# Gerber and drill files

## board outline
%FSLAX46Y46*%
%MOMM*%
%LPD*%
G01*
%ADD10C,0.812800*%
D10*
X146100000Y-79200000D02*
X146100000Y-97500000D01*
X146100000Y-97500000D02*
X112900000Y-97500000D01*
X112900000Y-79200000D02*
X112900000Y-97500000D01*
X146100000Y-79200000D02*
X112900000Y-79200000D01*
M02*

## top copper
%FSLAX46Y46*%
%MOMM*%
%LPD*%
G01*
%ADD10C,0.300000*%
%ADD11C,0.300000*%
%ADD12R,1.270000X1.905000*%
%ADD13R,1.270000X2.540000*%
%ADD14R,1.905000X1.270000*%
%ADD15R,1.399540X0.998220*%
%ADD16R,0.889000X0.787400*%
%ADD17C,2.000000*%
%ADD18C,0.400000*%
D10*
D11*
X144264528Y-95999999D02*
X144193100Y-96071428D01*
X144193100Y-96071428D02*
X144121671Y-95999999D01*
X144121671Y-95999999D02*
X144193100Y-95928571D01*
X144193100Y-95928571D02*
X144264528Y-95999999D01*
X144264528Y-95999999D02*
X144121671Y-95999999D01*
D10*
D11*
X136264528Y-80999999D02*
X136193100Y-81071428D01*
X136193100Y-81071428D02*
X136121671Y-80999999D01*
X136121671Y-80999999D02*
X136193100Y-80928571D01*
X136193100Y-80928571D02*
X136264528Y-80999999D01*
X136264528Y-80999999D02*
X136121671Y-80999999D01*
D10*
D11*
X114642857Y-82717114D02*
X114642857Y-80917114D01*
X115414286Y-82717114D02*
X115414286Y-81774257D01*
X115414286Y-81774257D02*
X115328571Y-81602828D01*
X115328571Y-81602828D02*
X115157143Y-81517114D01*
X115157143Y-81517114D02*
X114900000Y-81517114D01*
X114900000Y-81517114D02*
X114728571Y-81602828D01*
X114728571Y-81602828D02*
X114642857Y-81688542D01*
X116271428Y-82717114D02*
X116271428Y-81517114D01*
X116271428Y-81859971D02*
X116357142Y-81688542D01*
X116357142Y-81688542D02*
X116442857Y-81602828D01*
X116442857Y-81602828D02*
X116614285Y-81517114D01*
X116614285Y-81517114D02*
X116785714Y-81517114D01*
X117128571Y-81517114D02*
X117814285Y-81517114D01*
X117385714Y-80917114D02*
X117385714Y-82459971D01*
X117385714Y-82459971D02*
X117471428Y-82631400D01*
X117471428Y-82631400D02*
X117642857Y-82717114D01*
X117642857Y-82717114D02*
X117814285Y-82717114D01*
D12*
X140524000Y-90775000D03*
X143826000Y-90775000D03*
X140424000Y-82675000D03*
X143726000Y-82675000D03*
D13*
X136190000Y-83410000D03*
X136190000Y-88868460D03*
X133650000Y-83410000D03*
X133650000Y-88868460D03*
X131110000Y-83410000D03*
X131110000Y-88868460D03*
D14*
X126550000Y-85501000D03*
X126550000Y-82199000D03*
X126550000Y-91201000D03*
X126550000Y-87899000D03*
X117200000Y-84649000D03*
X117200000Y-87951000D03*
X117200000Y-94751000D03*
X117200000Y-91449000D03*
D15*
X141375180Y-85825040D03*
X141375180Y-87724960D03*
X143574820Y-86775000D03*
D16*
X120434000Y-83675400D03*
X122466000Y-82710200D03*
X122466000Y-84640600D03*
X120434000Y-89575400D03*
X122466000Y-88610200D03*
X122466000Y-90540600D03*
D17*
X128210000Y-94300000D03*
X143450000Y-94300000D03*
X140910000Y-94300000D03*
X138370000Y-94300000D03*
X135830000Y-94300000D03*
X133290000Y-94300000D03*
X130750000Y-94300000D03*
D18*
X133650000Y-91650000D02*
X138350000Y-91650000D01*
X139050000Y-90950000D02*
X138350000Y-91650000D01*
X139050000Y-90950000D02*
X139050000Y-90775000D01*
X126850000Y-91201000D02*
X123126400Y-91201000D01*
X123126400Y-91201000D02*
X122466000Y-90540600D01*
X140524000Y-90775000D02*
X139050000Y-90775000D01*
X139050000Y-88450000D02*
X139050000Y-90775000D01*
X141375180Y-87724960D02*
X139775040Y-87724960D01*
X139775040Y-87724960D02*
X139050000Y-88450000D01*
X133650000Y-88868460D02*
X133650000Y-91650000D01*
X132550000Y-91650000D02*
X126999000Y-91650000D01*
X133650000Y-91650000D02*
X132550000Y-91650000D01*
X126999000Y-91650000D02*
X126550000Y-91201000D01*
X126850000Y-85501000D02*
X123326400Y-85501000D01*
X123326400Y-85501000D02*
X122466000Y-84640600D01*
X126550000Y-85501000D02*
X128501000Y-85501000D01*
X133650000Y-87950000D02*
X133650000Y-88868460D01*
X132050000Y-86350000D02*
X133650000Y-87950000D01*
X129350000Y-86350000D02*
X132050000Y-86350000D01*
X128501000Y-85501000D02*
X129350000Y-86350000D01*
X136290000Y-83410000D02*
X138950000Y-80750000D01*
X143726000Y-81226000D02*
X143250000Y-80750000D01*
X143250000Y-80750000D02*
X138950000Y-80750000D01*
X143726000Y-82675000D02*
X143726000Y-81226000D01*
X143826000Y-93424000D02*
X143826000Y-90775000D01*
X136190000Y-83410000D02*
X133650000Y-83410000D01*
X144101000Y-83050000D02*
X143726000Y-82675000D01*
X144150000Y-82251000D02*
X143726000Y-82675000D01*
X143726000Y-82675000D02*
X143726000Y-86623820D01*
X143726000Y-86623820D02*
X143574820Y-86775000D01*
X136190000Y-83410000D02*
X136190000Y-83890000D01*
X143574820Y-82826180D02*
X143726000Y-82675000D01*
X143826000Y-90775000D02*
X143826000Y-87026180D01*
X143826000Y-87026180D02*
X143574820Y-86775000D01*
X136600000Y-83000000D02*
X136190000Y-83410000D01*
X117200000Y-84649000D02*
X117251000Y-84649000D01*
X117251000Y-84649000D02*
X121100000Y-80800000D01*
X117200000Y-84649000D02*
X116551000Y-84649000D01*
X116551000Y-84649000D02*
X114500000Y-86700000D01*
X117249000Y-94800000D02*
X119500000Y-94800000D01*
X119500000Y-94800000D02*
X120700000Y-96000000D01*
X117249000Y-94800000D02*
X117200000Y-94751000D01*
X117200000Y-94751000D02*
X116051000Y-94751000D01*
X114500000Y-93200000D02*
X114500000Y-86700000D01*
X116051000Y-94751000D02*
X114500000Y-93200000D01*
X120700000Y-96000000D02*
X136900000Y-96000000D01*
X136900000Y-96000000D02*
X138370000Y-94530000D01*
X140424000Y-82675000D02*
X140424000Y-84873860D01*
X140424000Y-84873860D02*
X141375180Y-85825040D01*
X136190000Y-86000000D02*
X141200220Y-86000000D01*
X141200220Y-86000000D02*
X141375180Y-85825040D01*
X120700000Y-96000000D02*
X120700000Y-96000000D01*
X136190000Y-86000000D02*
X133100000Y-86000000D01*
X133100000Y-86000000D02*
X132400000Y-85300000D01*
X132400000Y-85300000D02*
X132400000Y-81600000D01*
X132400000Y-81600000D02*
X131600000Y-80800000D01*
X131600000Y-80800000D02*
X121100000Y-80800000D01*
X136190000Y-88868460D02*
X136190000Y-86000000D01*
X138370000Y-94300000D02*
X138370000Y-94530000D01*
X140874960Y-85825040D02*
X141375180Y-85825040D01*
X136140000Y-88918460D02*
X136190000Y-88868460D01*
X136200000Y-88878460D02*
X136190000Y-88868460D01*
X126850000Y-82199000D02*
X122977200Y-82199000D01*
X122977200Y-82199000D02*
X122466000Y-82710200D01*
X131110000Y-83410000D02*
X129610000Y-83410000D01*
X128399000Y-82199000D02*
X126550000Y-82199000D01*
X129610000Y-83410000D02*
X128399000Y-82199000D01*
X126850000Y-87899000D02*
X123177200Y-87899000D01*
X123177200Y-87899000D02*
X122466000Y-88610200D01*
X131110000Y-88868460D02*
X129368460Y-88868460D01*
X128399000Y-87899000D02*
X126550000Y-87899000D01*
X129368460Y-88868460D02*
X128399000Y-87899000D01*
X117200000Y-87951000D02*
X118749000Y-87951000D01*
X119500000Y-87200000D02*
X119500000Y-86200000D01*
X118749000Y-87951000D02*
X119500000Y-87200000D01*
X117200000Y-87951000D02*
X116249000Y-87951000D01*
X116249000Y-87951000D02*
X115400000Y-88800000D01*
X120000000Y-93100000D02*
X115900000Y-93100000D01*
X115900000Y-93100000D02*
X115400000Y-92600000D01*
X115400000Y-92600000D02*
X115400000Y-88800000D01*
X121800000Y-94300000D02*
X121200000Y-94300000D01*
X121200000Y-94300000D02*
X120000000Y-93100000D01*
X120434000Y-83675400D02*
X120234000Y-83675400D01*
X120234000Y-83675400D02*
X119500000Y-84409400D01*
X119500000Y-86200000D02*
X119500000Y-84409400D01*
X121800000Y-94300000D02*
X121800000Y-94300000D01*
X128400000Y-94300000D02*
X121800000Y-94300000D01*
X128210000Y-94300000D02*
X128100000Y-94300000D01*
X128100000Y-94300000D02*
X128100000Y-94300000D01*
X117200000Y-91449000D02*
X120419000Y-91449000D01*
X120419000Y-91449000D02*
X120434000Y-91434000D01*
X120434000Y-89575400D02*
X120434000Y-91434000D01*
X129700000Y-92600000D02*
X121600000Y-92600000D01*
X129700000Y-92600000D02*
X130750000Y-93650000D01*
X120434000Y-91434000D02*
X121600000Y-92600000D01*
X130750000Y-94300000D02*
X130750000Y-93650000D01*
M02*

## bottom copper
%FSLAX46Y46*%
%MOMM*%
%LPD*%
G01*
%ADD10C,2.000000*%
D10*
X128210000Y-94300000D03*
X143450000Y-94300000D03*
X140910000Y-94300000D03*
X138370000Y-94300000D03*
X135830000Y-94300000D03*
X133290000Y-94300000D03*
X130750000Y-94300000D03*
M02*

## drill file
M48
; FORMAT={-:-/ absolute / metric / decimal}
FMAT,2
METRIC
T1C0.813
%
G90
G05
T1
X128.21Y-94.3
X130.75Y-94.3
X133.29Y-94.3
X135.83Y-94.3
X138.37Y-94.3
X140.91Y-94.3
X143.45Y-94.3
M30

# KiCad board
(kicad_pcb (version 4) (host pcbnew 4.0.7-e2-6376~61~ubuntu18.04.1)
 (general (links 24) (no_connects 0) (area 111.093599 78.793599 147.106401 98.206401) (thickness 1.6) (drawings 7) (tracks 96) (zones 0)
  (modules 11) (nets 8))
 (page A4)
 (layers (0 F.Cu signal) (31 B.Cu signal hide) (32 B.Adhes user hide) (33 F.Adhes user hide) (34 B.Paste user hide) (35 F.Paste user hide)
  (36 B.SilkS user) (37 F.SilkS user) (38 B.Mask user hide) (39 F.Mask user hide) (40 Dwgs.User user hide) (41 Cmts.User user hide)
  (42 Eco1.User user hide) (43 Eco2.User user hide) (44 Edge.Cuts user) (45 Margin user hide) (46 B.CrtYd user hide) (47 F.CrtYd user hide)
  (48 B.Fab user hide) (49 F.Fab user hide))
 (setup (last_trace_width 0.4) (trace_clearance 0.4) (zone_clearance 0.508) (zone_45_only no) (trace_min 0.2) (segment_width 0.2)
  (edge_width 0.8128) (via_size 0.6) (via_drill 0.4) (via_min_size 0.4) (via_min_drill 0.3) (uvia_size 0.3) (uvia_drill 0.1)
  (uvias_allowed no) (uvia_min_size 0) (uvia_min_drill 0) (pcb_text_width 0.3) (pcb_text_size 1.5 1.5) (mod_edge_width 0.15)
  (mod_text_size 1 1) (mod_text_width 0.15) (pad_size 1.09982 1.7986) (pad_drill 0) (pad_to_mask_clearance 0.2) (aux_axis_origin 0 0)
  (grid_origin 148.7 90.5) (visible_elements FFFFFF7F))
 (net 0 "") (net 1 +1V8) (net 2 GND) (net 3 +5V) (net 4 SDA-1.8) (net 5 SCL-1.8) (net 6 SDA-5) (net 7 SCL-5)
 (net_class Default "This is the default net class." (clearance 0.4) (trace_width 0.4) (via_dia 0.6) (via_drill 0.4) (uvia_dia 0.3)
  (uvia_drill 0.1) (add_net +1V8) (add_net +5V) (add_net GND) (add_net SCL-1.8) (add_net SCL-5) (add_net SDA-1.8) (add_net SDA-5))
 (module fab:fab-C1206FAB (layer F.Cu) (at 142.175 90.775)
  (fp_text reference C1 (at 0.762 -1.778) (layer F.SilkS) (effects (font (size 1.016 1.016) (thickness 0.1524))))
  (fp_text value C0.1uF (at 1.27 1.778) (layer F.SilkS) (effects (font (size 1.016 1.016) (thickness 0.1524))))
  (pad 1 smd rect (at -1.651 0) (size 1.27 1.905) (layers F.Cu F.Paste F.Mask) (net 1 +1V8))
  (pad 2 smd rect (at 1.651 0) (size 1.27 1.905) (layers F.Cu F.Paste F.Mask) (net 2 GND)))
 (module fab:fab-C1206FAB (layer F.Cu) (at 142.075 82.675)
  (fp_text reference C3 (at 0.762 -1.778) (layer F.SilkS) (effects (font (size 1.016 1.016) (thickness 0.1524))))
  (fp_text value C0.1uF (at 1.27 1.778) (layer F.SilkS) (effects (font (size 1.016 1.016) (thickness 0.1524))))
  (pad 1 smd rect (at -1.651 0) (size 1.27 1.905) (layers F.Cu F.Paste F.Mask) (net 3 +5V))
  (pad 2 smd rect (at 1.651 0) (size 1.27 1.905) (layers F.Cu F.Paste F.Mask) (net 2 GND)))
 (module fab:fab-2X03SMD (layer F.Cu) (at 133.65 85.95 270)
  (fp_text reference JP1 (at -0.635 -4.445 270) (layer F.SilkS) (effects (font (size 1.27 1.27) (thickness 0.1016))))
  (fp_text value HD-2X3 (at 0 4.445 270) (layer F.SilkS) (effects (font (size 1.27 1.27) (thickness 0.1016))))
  (pad 1 smd rect (at -2.54 -2.54 270) (size 2.54 1.27) (layers F.Cu F.Paste F.Mask) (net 2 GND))
  (pad 2 smd rect (at 2.91846 -2.54 270) (size 2.54 1.27) (layers F.Cu F.Paste F.Mask) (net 3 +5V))
  (pad 3 smd rect (at -2.54 0 270) (size 2.54 1.27) (layers F.Cu F.Paste F.Mask) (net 2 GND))
  (pad 4 smd rect (at 2.91846 0 270) (size 2.54 1.27) (layers F.Cu F.Paste F.Mask) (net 1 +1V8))
  (pad 5 smd rect (at -2.54 2.54 270) (size 2.54 1.27) (layers F.Cu F.Paste F.Mask) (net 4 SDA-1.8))
  (pad 6 smd rect (at 2.91846 2.54 270) (size 2.54 1.27) (layers F.Cu F.Paste F.Mask) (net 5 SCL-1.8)))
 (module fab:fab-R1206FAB (layer F.Cu) (at 126.55 83.85 90)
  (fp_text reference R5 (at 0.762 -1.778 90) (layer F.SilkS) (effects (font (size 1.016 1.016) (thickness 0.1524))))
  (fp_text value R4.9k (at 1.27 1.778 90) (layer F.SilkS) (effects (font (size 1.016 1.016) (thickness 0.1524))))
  (pad 1 smd rect (at -1.651 0 90) (size 1.27 1.905) (layers F.Cu F.Paste F.Mask) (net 1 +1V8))
  (pad 2 smd rect (at 1.651 0 90) (size 1.27 1.905) (layers F.Cu F.Paste F.Mask) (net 4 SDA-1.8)))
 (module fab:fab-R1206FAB (layer F.Cu) (at 126.55 89.55 90)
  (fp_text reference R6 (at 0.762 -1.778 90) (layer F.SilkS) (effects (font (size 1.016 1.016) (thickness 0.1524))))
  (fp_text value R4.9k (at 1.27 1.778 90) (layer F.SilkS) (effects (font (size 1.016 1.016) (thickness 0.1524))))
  (pad 1 smd rect (at -1.651 0 90) (size 1.27 1.905) (layers F.Cu F.Paste F.Mask) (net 1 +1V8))
  (pad 2 smd rect (at 1.651 0 90) (size 1.27 1.905) (layers F.Cu F.Paste F.Mask) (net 5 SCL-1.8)))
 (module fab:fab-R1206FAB (layer F.Cu) (at 117.2 86.3 270)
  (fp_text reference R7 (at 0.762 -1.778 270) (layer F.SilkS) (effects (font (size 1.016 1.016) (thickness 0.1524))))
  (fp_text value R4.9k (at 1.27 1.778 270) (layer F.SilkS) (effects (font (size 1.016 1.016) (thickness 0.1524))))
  (pad 1 smd rect (at -1.651 0 270) (size 1.27 1.905) (layers F.Cu F.Paste F.Mask) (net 3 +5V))
  (pad 2 smd rect (at 1.651 0 270) (size 1.27 1.905) (layers F.Cu F.Paste F.Mask) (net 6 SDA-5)))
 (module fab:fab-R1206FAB (layer F.Cu) (at 117.2 93.1 90)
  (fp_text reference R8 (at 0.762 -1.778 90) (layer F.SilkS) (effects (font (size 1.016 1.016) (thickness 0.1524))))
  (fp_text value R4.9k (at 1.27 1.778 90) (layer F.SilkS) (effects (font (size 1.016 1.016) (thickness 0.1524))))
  (pad 1 smd rect (at -1.651 0 90) (size 1.27 1.905) (layers F.Cu F.Paste F.Mask) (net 3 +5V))
  (pad 2 smd rect (at 1.651 0 90) (size 1.27 1.905) (layers F.Cu F.Paste F.Mask) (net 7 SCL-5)))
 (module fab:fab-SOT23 (layer F.Cu) (at 142.475 86.775 270)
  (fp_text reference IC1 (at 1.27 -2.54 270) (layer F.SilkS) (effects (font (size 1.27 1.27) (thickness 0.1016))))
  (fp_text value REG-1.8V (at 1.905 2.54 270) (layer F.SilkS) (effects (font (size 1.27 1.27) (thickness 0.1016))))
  (pad 1 smd rect (at -0.94996 1.09982 270) (size 0.99822 1.39954) (layers F.Cu F.Paste F.Mask) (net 3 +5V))
  (pad 2 smd rect (at 0.94996 1.09982 270) (size 0.99822 1.39954) (layers F.Cu F.Paste F.Mask) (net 1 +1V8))
  (pad 3 smd rect (at 0 -1.09982 270) (size 0.99822 1.39954) (layers F.Cu F.Paste F.Mask) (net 2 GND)))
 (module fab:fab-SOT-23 (layer F.Cu) (at 121.45 83.65 270)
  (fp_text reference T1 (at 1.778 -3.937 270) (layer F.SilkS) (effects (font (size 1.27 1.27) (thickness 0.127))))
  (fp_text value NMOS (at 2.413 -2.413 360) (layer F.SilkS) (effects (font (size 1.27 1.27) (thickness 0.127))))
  (pad 1 smd rect (at 0.0254 1.016 270) (size 0.7874 0.889) (layers F.Cu F.Paste F.Mask) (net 6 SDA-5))
  (pad 2 smd rect (at -0.9398 -1.016 270) (size 0.7874 0.889) (layers F.Cu F.Paste F.Mask) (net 4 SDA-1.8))
  (pad 3 smd rect (at 0.9906 -1.016 270) (size 0.7874 0.889) (layers F.Cu F.Paste F.Mask) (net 1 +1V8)))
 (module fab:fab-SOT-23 (layer F.Cu) (at 121.45 89.55 270)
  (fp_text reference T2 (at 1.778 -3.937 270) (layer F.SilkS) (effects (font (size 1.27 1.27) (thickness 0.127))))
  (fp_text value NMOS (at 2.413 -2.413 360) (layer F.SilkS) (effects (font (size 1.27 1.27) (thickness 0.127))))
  (pad 1 smd rect (at 0.0254 1.016 270) (size 0.7874 0.889) (layers F.Cu F.Paste F.Mask) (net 7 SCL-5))
  (pad 2 smd rect (at -0.9398 -1.016 270) (size 0.7874 0.889) (layers F.Cu F.Paste F.Mask) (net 5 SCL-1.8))
  (pad 3 smd rect (at 0.9906 -1.016 270) (size 0.7874 0.889) (layers F.Cu F.Paste F.Mask) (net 1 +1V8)))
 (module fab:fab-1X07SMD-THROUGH (layer F.Cu) (at 137.1 94.3 270)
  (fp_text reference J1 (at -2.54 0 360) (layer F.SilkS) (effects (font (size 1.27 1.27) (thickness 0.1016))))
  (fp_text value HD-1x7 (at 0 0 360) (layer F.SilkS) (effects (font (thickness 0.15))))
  (pad 7 thru_hole circle (at 0 8.89 270) (size 2 2) (drill 0.8128) (layers F.Cu F.Paste F.Mask) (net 6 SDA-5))
  (pad 1 thru_hole circle (at 0 -6.35 270) (size 2 2) (drill 0.8128) (layers F.Cu F.Paste F.Mask) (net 2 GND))
  (pad 2 thru_hole circle (at 0 -3.81 270) (size 2 2) (drill 0.8128) (layers F.Cu F.Paste F.Mask))
  (pad 3 thru_hole circle (at 0 -1.27 270) (size 2 2) (drill 0.8128) (layers F.Cu F.Paste F.Mask) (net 3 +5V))
  (pad 4 thru_hole circle (at 0 1.27 270) (size 2 2) (drill 0.8128) (layers F.Cu F.Paste F.Mask))
  (pad 5 thru_hole circle (at 0 3.81 270) (size 2 2) (drill 0.8128) (layers F.Cu F.Paste F.Mask))
  (pad 6 thru_hole circle (at 0 6.35 270) (size 2 2) (drill 0.8128) (layers F.Cu F.Paste F.Mask) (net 7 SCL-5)))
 (gr_line (start 146.1 79.2) (end 146.1 97.5) (angle 90) (layer Edge.Cuts) (width 0.8128))
 (gr_line (start 146.1 97.5) (end 112.9 97.5) (angle 90) (layer Edge.Cuts) (width 0.8128))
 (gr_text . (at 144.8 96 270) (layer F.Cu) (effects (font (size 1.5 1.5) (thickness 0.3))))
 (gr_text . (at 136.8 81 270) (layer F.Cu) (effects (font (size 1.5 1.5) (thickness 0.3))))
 (gr_line (start 112.9 79.2) (end 112.9 97.5) (angle 90) (layer Edge.Cuts) (width 0.8128))
 (gr_line (start 146.1 79.2) (end 112.9 79.2) (angle 90) (layer Edge.Cuts) (width 0.8128))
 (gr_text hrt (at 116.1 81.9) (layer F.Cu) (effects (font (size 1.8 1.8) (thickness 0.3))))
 (segment (start 133.65 91.65) (end 138.35 91.65) (width 0.4) (layer F.Cu) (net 1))
 (segment (start 139.05 90.95) (end 138.35 91.65) (width 0.4) (layer F.Cu) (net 1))
 (segment (start 139.05 90.95) (end 139.05 90.775) (width 0.4) (layer F.Cu) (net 1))
 (segment (start 126.85 91.201) (end 123.1264 91.201) (width 0.4) (layer F.Cu) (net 1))
 (segment (start 123.1264 91.201) (end 122.466 90.5406) (width 0.4) (layer F.Cu) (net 1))
 (segment (start 140.524 90.775) (end 139.05 90.775) (width 0.4) (layer F.Cu) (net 1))
 (segment (start 139.05 88.45) (end 139.05 90.775) (width 0.4) (layer F.Cu) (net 1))
 (segment (start 141.37518 87.72496) (end 139.77504 87.72496) (width 0.4) (layer F.Cu) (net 1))
 (segment (start 139.77504 87.72496) (end 139.05 88.45) (width 0.4) (layer F.Cu) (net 1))
 (segment (start 133.65 88.86846) (end 133.65 91.65) (width 0.4) (layer F.Cu) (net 1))
 (segment (start 132.55 91.65) (end 126.999 91.65) (width 0.4) (layer F.Cu) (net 1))
 (segment (start 133.65 91.65) (end 132.55 91.65) (width 0.4) (layer F.Cu) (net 1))
 (segment (start 126.999 91.65) (end 126.55 91.201) (width 0.4) (layer F.Cu) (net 1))
 (segment (start 126.85 85.501) (end 123.3264 85.501) (width 0.4) (layer F.Cu) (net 1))
 (segment (start 123.3264 85.501) (end 122.466 84.6406) (width 0.4) (layer F.Cu) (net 1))
 (segment (start 126.55 85.501) (end 128.501 85.501) (width 0.4) (layer F.Cu) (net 1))
 (segment (start 133.65 87.95) (end 133.65 88.86846) (width 0.4) (layer F.Cu) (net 1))
 (segment (start 132.05 86.35) (end 133.65 87.95) (width 0.4) (layer F.Cu) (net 1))
 (segment (start 129.35 86.35) (end 132.05 86.35) (width 0.4) (layer F.Cu) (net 1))
 (segment (start 128.501 85.501) (end 129.35 86.35) (width 0.4) (layer F.Cu) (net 1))
 (segment (start 136.29 83.41) (end 138.95 80.75) (width 0.4) (layer F.Cu) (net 2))
 (segment (start 143.726 81.226) (end 143.25 80.75) (width 0.4) (layer F.Cu) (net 2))
 (segment (start 143.25 80.75) (end 138.95 80.75) (width 0.4) (layer F.Cu) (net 2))
 (segment (start 143.726 82.675) (end 143.726 81.226) (width 0.4) (layer F.Cu) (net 2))
 (segment (start 143.826 93.424) (end 143.826 90.775) (width 0.4) (layer F.Cu) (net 2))
 (segment (start 136.19 83.41) (end 133.65 83.41) (width 0.4) (layer F.Cu) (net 2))
 (segment (start 144.101 83.05) (end 143.726 82.675) (width 0.4) (layer F.Cu) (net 2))
 (segment (start 144.15 82.251) (end 143.726 82.675) (width 0.4) (layer F.Cu) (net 2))
 (segment (start 143.726 82.675) (end 143.726 86.62382) (width 0.4) (layer F.Cu) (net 2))
 (segment (start 143.726 86.62382) (end 143.57482 86.775) (width 0.4) (layer F.Cu) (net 2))
 (segment (start 136.19 83.41) (end 136.19 83.89) (width 0.4) (layer F.Cu) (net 2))
 (segment (start 143.57482 82.82618) (end 143.726 82.675) (width 0.4) (layer F.Cu) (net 2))
 (segment (start 143.826 90.775) (end 143.826 87.02618) (width 0.4) (layer F.Cu) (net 2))
 (segment (start 143.826 87.02618) (end 143.57482 86.775) (width 0.4) (layer F.Cu) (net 2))
 (segment (start 136.6 83) (end 136.19 83.41) (width 0.4) (layer F.Cu) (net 2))
 (segment (start 117.2 84.649) (end 117.251 84.649) (width 0.4) (layer F.Cu) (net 3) (status C00000))
 (segment (start 117.251 84.649) (end 121.1 80.8) (width 0.4) (layer F.Cu) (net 3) (status 400000))
 (segment (start 117.2 84.649) (end 116.551 84.649) (width 0.4) (layer F.Cu) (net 3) (status C00000))
 (segment (start 116.551 84.649) (end 114.5 86.7) (width 0.4) (layer F.Cu) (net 3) (status 400000))
 (segment (start 117.249 94.8) (end 119.5 94.8) (width 0.4) (layer F.Cu) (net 3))
 (segment (start 119.5 94.8) (end 120.7 96) (width 0.4) (layer F.Cu) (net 3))
 (segment (start 117.249 94.8) (end 117.2 94.751) (width 0.4) (layer F.Cu) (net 3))
 (segment (start 117.2 94.751) (end 116.051 94.751) (width 0.4) (layer F.Cu) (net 3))
 (segment (start 114.5 93.2) (end 114.5 86.7) (width 0.4) (layer F.Cu) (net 3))
 (segment (start 116.051 94.751) (end 114.5 93.2) (width 0.4) (layer F.Cu) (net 3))
 (segment (start 120.7 96) (end 136.9 96) (width 0.4) (layer F.Cu) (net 3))
 (segment (start 136.9 96) (end 138.37 94.53) (width 0.4) (layer F.Cu) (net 3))
 (segment (start 140.424 82.675) (end 140.424 84.87386) (width 0.4) (layer F.Cu) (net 3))
 (segment (start 140.424 84.87386) (end 141.37518 85.82504) (width 0.4) (layer F.Cu) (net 3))
 (segment (start 136.19 86) (end 141.20022 86) (width 0.4) (layer F.Cu) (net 3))
 (segment (start 141.20022 86) (end 141.37518 85.82504) (width 0.4) (layer F.Cu) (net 3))
 (segment (start 120.7 96) (end 120.7 96) (width 0.4) (layer F.Cu) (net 3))
 (segment (start 136.19 86) (end 133.1 86) (width 0.4) (layer F.Cu) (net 3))
 (segment (start 133.1 86) (end 132.4 85.3) (width 0.4) (layer F.Cu) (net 3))
 (segment (start 132.4 85.3) (end 132.4 81.6) (width 0.4) (layer F.Cu) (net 3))
 (segment (start 132.4 81.6) (end 131.6 80.8) (width 0.4) (layer F.Cu) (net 3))
 (segment (start 131.6 80.8) (end 121.1 80.8) (width 0.4) (layer F.Cu) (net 3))
 (segment (start 136.19 88.86846) (end 136.19 86) (width 0.4) (layer F.Cu) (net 3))
 (segment (start 138.37 94.3) (end 138.37 94.53) (width 0.4) (layer F.Cu) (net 3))
 (segment (start 140.87496 85.82504) (end 141.37518 85.82504) (width 0.4) (layer F.Cu) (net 3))
 (segment (start 136.14 88.91846) (end 136.19 88.86846) (width 0.4) (layer F.Cu) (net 3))
 (segment (start 136.2 88.87846) (end 136.19 88.86846) (width 0.4) (layer F.Cu) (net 3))
 (segment (start 126.85 82.199) (end 122.9772 82.199) (width 0.4) (layer F.Cu) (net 4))
 (segment (start 122.9772 82.199) (end 122.466 82.7102) (width 0.4) (layer F.Cu) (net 4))
 (segment (start 131.11 83.41) (end 129.61 83.41) (width 0.4) (layer F.Cu) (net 4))
 (segment (start 128.399 82.199) (end 126.55 82.199) (width 0.4) (layer F.Cu) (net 4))
 (segment (start 129.61 83.41) (end 128.399 82.199) (width 0.4) (layer F.Cu) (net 4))
 (segment (start 126.85 87.899) (end 123.1772 87.899) (width 0.4) (layer F.Cu) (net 5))
 (segment (start 123.1772 87.899) (end 122.466 88.6102) (width 0.4) (layer F.Cu) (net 5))
 (segment (start 131.11 88.86846) (end 129.36846 88.86846) (width 0.4) (layer F.Cu) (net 5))
 (segment (start 128.399 87.899) (end 126.55 87.899) (width 0.4) (layer F.Cu) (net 5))
 (segment (start 129.36846 88.86846) (end 128.399 87.899) (width 0.4) (layer F.Cu) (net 5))
 (segment (start 117.2 87.951) (end 118.749 87.951) (width 0.4) (layer F.Cu) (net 6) (status 400000))
 (segment (start 119.5 87.2) (end 119.5 86.2) (width 0.4) (layer F.Cu) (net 6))
 (segment (start 118.749 87.951) (end 119.5 87.2) (width 0.4) (layer F.Cu) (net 6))
 (segment (start 117.2 87.951) (end 116.249 87.951) (width 0.4) (layer F.Cu) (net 6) (status C00000))
 (segment (start 116.249 87.951) (end 115.4 88.8) (width 0.4) (layer F.Cu) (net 6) (status 400000))
 (segment (start 120 93.1) (end 115.9 93.1) (width 0.4) (layer F.Cu) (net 6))
 (segment (start 115.9 93.1) (end 115.4 92.6) (width 0.4) (layer F.Cu) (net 6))
 (segment (start 115.4 92.6) (end 115.4 88.8) (width 0.4) (layer F.Cu) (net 6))
 (segment (start 121.8 94.3) (end 121.2 94.3) (width 0.4) (layer F.Cu) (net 6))
 (segment (start 121.2 94.3) (end 120 93.1) (width 0.4) (layer F.Cu) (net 6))
 (segment (start 120.434 83.6754) (end 120.234 83.6754) (width 0.4) (layer F.Cu) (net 6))
 (segment (start 120.234 83.6754) (end 119.5 84.4094) (width 0.4) (layer F.Cu) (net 6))
 (segment (start 119.5 86.2) (end 119.5 84.4094) (width 0.4) (layer F.Cu) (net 6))
 (segment (start 121.8 94.3) (end 121.8 94.3) (width 0.4) (layer F.Cu) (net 6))
 (segment (start 128.4 94.3) (end 121.8 94.3) (width 0.4) (layer F.Cu) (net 6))
 (segment (start 128.21 94.3) (end 128.1 94.3) (width 0.4) (layer F.Cu) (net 6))
 (segment (start 128.1 94.3) (end 128.1 94.3) (width 0.4) (layer F.Cu) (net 6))
 (segment (start 117.2 91.449) (end 120.419 91.449) (width 0.4) (layer F.Cu) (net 7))
 (segment (start 120.419 91.449) (end 120.434 91.434) (width 0.4) (layer F.Cu) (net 7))
 (segment (start 120.434 89.5754) (end 120.434 91.434) (width 0.4) (layer F.Cu) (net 7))
 (segment (start 129.7 92.6) (end 121.6 92.6) (width 0.4) (layer F.Cu) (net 7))
 (segment (start 129.7 92.6) (end 130.75 93.65) (width 0.4) (layer F.Cu) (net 7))
 (segment (start 120.434 91.434) (end 121.6 92.6) (width 0.4) (layer F.Cu) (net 7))
 (segment (start 130.75 94.3) (end 130.75 93.65) (width 0.4) (layer F.Cu) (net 7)))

